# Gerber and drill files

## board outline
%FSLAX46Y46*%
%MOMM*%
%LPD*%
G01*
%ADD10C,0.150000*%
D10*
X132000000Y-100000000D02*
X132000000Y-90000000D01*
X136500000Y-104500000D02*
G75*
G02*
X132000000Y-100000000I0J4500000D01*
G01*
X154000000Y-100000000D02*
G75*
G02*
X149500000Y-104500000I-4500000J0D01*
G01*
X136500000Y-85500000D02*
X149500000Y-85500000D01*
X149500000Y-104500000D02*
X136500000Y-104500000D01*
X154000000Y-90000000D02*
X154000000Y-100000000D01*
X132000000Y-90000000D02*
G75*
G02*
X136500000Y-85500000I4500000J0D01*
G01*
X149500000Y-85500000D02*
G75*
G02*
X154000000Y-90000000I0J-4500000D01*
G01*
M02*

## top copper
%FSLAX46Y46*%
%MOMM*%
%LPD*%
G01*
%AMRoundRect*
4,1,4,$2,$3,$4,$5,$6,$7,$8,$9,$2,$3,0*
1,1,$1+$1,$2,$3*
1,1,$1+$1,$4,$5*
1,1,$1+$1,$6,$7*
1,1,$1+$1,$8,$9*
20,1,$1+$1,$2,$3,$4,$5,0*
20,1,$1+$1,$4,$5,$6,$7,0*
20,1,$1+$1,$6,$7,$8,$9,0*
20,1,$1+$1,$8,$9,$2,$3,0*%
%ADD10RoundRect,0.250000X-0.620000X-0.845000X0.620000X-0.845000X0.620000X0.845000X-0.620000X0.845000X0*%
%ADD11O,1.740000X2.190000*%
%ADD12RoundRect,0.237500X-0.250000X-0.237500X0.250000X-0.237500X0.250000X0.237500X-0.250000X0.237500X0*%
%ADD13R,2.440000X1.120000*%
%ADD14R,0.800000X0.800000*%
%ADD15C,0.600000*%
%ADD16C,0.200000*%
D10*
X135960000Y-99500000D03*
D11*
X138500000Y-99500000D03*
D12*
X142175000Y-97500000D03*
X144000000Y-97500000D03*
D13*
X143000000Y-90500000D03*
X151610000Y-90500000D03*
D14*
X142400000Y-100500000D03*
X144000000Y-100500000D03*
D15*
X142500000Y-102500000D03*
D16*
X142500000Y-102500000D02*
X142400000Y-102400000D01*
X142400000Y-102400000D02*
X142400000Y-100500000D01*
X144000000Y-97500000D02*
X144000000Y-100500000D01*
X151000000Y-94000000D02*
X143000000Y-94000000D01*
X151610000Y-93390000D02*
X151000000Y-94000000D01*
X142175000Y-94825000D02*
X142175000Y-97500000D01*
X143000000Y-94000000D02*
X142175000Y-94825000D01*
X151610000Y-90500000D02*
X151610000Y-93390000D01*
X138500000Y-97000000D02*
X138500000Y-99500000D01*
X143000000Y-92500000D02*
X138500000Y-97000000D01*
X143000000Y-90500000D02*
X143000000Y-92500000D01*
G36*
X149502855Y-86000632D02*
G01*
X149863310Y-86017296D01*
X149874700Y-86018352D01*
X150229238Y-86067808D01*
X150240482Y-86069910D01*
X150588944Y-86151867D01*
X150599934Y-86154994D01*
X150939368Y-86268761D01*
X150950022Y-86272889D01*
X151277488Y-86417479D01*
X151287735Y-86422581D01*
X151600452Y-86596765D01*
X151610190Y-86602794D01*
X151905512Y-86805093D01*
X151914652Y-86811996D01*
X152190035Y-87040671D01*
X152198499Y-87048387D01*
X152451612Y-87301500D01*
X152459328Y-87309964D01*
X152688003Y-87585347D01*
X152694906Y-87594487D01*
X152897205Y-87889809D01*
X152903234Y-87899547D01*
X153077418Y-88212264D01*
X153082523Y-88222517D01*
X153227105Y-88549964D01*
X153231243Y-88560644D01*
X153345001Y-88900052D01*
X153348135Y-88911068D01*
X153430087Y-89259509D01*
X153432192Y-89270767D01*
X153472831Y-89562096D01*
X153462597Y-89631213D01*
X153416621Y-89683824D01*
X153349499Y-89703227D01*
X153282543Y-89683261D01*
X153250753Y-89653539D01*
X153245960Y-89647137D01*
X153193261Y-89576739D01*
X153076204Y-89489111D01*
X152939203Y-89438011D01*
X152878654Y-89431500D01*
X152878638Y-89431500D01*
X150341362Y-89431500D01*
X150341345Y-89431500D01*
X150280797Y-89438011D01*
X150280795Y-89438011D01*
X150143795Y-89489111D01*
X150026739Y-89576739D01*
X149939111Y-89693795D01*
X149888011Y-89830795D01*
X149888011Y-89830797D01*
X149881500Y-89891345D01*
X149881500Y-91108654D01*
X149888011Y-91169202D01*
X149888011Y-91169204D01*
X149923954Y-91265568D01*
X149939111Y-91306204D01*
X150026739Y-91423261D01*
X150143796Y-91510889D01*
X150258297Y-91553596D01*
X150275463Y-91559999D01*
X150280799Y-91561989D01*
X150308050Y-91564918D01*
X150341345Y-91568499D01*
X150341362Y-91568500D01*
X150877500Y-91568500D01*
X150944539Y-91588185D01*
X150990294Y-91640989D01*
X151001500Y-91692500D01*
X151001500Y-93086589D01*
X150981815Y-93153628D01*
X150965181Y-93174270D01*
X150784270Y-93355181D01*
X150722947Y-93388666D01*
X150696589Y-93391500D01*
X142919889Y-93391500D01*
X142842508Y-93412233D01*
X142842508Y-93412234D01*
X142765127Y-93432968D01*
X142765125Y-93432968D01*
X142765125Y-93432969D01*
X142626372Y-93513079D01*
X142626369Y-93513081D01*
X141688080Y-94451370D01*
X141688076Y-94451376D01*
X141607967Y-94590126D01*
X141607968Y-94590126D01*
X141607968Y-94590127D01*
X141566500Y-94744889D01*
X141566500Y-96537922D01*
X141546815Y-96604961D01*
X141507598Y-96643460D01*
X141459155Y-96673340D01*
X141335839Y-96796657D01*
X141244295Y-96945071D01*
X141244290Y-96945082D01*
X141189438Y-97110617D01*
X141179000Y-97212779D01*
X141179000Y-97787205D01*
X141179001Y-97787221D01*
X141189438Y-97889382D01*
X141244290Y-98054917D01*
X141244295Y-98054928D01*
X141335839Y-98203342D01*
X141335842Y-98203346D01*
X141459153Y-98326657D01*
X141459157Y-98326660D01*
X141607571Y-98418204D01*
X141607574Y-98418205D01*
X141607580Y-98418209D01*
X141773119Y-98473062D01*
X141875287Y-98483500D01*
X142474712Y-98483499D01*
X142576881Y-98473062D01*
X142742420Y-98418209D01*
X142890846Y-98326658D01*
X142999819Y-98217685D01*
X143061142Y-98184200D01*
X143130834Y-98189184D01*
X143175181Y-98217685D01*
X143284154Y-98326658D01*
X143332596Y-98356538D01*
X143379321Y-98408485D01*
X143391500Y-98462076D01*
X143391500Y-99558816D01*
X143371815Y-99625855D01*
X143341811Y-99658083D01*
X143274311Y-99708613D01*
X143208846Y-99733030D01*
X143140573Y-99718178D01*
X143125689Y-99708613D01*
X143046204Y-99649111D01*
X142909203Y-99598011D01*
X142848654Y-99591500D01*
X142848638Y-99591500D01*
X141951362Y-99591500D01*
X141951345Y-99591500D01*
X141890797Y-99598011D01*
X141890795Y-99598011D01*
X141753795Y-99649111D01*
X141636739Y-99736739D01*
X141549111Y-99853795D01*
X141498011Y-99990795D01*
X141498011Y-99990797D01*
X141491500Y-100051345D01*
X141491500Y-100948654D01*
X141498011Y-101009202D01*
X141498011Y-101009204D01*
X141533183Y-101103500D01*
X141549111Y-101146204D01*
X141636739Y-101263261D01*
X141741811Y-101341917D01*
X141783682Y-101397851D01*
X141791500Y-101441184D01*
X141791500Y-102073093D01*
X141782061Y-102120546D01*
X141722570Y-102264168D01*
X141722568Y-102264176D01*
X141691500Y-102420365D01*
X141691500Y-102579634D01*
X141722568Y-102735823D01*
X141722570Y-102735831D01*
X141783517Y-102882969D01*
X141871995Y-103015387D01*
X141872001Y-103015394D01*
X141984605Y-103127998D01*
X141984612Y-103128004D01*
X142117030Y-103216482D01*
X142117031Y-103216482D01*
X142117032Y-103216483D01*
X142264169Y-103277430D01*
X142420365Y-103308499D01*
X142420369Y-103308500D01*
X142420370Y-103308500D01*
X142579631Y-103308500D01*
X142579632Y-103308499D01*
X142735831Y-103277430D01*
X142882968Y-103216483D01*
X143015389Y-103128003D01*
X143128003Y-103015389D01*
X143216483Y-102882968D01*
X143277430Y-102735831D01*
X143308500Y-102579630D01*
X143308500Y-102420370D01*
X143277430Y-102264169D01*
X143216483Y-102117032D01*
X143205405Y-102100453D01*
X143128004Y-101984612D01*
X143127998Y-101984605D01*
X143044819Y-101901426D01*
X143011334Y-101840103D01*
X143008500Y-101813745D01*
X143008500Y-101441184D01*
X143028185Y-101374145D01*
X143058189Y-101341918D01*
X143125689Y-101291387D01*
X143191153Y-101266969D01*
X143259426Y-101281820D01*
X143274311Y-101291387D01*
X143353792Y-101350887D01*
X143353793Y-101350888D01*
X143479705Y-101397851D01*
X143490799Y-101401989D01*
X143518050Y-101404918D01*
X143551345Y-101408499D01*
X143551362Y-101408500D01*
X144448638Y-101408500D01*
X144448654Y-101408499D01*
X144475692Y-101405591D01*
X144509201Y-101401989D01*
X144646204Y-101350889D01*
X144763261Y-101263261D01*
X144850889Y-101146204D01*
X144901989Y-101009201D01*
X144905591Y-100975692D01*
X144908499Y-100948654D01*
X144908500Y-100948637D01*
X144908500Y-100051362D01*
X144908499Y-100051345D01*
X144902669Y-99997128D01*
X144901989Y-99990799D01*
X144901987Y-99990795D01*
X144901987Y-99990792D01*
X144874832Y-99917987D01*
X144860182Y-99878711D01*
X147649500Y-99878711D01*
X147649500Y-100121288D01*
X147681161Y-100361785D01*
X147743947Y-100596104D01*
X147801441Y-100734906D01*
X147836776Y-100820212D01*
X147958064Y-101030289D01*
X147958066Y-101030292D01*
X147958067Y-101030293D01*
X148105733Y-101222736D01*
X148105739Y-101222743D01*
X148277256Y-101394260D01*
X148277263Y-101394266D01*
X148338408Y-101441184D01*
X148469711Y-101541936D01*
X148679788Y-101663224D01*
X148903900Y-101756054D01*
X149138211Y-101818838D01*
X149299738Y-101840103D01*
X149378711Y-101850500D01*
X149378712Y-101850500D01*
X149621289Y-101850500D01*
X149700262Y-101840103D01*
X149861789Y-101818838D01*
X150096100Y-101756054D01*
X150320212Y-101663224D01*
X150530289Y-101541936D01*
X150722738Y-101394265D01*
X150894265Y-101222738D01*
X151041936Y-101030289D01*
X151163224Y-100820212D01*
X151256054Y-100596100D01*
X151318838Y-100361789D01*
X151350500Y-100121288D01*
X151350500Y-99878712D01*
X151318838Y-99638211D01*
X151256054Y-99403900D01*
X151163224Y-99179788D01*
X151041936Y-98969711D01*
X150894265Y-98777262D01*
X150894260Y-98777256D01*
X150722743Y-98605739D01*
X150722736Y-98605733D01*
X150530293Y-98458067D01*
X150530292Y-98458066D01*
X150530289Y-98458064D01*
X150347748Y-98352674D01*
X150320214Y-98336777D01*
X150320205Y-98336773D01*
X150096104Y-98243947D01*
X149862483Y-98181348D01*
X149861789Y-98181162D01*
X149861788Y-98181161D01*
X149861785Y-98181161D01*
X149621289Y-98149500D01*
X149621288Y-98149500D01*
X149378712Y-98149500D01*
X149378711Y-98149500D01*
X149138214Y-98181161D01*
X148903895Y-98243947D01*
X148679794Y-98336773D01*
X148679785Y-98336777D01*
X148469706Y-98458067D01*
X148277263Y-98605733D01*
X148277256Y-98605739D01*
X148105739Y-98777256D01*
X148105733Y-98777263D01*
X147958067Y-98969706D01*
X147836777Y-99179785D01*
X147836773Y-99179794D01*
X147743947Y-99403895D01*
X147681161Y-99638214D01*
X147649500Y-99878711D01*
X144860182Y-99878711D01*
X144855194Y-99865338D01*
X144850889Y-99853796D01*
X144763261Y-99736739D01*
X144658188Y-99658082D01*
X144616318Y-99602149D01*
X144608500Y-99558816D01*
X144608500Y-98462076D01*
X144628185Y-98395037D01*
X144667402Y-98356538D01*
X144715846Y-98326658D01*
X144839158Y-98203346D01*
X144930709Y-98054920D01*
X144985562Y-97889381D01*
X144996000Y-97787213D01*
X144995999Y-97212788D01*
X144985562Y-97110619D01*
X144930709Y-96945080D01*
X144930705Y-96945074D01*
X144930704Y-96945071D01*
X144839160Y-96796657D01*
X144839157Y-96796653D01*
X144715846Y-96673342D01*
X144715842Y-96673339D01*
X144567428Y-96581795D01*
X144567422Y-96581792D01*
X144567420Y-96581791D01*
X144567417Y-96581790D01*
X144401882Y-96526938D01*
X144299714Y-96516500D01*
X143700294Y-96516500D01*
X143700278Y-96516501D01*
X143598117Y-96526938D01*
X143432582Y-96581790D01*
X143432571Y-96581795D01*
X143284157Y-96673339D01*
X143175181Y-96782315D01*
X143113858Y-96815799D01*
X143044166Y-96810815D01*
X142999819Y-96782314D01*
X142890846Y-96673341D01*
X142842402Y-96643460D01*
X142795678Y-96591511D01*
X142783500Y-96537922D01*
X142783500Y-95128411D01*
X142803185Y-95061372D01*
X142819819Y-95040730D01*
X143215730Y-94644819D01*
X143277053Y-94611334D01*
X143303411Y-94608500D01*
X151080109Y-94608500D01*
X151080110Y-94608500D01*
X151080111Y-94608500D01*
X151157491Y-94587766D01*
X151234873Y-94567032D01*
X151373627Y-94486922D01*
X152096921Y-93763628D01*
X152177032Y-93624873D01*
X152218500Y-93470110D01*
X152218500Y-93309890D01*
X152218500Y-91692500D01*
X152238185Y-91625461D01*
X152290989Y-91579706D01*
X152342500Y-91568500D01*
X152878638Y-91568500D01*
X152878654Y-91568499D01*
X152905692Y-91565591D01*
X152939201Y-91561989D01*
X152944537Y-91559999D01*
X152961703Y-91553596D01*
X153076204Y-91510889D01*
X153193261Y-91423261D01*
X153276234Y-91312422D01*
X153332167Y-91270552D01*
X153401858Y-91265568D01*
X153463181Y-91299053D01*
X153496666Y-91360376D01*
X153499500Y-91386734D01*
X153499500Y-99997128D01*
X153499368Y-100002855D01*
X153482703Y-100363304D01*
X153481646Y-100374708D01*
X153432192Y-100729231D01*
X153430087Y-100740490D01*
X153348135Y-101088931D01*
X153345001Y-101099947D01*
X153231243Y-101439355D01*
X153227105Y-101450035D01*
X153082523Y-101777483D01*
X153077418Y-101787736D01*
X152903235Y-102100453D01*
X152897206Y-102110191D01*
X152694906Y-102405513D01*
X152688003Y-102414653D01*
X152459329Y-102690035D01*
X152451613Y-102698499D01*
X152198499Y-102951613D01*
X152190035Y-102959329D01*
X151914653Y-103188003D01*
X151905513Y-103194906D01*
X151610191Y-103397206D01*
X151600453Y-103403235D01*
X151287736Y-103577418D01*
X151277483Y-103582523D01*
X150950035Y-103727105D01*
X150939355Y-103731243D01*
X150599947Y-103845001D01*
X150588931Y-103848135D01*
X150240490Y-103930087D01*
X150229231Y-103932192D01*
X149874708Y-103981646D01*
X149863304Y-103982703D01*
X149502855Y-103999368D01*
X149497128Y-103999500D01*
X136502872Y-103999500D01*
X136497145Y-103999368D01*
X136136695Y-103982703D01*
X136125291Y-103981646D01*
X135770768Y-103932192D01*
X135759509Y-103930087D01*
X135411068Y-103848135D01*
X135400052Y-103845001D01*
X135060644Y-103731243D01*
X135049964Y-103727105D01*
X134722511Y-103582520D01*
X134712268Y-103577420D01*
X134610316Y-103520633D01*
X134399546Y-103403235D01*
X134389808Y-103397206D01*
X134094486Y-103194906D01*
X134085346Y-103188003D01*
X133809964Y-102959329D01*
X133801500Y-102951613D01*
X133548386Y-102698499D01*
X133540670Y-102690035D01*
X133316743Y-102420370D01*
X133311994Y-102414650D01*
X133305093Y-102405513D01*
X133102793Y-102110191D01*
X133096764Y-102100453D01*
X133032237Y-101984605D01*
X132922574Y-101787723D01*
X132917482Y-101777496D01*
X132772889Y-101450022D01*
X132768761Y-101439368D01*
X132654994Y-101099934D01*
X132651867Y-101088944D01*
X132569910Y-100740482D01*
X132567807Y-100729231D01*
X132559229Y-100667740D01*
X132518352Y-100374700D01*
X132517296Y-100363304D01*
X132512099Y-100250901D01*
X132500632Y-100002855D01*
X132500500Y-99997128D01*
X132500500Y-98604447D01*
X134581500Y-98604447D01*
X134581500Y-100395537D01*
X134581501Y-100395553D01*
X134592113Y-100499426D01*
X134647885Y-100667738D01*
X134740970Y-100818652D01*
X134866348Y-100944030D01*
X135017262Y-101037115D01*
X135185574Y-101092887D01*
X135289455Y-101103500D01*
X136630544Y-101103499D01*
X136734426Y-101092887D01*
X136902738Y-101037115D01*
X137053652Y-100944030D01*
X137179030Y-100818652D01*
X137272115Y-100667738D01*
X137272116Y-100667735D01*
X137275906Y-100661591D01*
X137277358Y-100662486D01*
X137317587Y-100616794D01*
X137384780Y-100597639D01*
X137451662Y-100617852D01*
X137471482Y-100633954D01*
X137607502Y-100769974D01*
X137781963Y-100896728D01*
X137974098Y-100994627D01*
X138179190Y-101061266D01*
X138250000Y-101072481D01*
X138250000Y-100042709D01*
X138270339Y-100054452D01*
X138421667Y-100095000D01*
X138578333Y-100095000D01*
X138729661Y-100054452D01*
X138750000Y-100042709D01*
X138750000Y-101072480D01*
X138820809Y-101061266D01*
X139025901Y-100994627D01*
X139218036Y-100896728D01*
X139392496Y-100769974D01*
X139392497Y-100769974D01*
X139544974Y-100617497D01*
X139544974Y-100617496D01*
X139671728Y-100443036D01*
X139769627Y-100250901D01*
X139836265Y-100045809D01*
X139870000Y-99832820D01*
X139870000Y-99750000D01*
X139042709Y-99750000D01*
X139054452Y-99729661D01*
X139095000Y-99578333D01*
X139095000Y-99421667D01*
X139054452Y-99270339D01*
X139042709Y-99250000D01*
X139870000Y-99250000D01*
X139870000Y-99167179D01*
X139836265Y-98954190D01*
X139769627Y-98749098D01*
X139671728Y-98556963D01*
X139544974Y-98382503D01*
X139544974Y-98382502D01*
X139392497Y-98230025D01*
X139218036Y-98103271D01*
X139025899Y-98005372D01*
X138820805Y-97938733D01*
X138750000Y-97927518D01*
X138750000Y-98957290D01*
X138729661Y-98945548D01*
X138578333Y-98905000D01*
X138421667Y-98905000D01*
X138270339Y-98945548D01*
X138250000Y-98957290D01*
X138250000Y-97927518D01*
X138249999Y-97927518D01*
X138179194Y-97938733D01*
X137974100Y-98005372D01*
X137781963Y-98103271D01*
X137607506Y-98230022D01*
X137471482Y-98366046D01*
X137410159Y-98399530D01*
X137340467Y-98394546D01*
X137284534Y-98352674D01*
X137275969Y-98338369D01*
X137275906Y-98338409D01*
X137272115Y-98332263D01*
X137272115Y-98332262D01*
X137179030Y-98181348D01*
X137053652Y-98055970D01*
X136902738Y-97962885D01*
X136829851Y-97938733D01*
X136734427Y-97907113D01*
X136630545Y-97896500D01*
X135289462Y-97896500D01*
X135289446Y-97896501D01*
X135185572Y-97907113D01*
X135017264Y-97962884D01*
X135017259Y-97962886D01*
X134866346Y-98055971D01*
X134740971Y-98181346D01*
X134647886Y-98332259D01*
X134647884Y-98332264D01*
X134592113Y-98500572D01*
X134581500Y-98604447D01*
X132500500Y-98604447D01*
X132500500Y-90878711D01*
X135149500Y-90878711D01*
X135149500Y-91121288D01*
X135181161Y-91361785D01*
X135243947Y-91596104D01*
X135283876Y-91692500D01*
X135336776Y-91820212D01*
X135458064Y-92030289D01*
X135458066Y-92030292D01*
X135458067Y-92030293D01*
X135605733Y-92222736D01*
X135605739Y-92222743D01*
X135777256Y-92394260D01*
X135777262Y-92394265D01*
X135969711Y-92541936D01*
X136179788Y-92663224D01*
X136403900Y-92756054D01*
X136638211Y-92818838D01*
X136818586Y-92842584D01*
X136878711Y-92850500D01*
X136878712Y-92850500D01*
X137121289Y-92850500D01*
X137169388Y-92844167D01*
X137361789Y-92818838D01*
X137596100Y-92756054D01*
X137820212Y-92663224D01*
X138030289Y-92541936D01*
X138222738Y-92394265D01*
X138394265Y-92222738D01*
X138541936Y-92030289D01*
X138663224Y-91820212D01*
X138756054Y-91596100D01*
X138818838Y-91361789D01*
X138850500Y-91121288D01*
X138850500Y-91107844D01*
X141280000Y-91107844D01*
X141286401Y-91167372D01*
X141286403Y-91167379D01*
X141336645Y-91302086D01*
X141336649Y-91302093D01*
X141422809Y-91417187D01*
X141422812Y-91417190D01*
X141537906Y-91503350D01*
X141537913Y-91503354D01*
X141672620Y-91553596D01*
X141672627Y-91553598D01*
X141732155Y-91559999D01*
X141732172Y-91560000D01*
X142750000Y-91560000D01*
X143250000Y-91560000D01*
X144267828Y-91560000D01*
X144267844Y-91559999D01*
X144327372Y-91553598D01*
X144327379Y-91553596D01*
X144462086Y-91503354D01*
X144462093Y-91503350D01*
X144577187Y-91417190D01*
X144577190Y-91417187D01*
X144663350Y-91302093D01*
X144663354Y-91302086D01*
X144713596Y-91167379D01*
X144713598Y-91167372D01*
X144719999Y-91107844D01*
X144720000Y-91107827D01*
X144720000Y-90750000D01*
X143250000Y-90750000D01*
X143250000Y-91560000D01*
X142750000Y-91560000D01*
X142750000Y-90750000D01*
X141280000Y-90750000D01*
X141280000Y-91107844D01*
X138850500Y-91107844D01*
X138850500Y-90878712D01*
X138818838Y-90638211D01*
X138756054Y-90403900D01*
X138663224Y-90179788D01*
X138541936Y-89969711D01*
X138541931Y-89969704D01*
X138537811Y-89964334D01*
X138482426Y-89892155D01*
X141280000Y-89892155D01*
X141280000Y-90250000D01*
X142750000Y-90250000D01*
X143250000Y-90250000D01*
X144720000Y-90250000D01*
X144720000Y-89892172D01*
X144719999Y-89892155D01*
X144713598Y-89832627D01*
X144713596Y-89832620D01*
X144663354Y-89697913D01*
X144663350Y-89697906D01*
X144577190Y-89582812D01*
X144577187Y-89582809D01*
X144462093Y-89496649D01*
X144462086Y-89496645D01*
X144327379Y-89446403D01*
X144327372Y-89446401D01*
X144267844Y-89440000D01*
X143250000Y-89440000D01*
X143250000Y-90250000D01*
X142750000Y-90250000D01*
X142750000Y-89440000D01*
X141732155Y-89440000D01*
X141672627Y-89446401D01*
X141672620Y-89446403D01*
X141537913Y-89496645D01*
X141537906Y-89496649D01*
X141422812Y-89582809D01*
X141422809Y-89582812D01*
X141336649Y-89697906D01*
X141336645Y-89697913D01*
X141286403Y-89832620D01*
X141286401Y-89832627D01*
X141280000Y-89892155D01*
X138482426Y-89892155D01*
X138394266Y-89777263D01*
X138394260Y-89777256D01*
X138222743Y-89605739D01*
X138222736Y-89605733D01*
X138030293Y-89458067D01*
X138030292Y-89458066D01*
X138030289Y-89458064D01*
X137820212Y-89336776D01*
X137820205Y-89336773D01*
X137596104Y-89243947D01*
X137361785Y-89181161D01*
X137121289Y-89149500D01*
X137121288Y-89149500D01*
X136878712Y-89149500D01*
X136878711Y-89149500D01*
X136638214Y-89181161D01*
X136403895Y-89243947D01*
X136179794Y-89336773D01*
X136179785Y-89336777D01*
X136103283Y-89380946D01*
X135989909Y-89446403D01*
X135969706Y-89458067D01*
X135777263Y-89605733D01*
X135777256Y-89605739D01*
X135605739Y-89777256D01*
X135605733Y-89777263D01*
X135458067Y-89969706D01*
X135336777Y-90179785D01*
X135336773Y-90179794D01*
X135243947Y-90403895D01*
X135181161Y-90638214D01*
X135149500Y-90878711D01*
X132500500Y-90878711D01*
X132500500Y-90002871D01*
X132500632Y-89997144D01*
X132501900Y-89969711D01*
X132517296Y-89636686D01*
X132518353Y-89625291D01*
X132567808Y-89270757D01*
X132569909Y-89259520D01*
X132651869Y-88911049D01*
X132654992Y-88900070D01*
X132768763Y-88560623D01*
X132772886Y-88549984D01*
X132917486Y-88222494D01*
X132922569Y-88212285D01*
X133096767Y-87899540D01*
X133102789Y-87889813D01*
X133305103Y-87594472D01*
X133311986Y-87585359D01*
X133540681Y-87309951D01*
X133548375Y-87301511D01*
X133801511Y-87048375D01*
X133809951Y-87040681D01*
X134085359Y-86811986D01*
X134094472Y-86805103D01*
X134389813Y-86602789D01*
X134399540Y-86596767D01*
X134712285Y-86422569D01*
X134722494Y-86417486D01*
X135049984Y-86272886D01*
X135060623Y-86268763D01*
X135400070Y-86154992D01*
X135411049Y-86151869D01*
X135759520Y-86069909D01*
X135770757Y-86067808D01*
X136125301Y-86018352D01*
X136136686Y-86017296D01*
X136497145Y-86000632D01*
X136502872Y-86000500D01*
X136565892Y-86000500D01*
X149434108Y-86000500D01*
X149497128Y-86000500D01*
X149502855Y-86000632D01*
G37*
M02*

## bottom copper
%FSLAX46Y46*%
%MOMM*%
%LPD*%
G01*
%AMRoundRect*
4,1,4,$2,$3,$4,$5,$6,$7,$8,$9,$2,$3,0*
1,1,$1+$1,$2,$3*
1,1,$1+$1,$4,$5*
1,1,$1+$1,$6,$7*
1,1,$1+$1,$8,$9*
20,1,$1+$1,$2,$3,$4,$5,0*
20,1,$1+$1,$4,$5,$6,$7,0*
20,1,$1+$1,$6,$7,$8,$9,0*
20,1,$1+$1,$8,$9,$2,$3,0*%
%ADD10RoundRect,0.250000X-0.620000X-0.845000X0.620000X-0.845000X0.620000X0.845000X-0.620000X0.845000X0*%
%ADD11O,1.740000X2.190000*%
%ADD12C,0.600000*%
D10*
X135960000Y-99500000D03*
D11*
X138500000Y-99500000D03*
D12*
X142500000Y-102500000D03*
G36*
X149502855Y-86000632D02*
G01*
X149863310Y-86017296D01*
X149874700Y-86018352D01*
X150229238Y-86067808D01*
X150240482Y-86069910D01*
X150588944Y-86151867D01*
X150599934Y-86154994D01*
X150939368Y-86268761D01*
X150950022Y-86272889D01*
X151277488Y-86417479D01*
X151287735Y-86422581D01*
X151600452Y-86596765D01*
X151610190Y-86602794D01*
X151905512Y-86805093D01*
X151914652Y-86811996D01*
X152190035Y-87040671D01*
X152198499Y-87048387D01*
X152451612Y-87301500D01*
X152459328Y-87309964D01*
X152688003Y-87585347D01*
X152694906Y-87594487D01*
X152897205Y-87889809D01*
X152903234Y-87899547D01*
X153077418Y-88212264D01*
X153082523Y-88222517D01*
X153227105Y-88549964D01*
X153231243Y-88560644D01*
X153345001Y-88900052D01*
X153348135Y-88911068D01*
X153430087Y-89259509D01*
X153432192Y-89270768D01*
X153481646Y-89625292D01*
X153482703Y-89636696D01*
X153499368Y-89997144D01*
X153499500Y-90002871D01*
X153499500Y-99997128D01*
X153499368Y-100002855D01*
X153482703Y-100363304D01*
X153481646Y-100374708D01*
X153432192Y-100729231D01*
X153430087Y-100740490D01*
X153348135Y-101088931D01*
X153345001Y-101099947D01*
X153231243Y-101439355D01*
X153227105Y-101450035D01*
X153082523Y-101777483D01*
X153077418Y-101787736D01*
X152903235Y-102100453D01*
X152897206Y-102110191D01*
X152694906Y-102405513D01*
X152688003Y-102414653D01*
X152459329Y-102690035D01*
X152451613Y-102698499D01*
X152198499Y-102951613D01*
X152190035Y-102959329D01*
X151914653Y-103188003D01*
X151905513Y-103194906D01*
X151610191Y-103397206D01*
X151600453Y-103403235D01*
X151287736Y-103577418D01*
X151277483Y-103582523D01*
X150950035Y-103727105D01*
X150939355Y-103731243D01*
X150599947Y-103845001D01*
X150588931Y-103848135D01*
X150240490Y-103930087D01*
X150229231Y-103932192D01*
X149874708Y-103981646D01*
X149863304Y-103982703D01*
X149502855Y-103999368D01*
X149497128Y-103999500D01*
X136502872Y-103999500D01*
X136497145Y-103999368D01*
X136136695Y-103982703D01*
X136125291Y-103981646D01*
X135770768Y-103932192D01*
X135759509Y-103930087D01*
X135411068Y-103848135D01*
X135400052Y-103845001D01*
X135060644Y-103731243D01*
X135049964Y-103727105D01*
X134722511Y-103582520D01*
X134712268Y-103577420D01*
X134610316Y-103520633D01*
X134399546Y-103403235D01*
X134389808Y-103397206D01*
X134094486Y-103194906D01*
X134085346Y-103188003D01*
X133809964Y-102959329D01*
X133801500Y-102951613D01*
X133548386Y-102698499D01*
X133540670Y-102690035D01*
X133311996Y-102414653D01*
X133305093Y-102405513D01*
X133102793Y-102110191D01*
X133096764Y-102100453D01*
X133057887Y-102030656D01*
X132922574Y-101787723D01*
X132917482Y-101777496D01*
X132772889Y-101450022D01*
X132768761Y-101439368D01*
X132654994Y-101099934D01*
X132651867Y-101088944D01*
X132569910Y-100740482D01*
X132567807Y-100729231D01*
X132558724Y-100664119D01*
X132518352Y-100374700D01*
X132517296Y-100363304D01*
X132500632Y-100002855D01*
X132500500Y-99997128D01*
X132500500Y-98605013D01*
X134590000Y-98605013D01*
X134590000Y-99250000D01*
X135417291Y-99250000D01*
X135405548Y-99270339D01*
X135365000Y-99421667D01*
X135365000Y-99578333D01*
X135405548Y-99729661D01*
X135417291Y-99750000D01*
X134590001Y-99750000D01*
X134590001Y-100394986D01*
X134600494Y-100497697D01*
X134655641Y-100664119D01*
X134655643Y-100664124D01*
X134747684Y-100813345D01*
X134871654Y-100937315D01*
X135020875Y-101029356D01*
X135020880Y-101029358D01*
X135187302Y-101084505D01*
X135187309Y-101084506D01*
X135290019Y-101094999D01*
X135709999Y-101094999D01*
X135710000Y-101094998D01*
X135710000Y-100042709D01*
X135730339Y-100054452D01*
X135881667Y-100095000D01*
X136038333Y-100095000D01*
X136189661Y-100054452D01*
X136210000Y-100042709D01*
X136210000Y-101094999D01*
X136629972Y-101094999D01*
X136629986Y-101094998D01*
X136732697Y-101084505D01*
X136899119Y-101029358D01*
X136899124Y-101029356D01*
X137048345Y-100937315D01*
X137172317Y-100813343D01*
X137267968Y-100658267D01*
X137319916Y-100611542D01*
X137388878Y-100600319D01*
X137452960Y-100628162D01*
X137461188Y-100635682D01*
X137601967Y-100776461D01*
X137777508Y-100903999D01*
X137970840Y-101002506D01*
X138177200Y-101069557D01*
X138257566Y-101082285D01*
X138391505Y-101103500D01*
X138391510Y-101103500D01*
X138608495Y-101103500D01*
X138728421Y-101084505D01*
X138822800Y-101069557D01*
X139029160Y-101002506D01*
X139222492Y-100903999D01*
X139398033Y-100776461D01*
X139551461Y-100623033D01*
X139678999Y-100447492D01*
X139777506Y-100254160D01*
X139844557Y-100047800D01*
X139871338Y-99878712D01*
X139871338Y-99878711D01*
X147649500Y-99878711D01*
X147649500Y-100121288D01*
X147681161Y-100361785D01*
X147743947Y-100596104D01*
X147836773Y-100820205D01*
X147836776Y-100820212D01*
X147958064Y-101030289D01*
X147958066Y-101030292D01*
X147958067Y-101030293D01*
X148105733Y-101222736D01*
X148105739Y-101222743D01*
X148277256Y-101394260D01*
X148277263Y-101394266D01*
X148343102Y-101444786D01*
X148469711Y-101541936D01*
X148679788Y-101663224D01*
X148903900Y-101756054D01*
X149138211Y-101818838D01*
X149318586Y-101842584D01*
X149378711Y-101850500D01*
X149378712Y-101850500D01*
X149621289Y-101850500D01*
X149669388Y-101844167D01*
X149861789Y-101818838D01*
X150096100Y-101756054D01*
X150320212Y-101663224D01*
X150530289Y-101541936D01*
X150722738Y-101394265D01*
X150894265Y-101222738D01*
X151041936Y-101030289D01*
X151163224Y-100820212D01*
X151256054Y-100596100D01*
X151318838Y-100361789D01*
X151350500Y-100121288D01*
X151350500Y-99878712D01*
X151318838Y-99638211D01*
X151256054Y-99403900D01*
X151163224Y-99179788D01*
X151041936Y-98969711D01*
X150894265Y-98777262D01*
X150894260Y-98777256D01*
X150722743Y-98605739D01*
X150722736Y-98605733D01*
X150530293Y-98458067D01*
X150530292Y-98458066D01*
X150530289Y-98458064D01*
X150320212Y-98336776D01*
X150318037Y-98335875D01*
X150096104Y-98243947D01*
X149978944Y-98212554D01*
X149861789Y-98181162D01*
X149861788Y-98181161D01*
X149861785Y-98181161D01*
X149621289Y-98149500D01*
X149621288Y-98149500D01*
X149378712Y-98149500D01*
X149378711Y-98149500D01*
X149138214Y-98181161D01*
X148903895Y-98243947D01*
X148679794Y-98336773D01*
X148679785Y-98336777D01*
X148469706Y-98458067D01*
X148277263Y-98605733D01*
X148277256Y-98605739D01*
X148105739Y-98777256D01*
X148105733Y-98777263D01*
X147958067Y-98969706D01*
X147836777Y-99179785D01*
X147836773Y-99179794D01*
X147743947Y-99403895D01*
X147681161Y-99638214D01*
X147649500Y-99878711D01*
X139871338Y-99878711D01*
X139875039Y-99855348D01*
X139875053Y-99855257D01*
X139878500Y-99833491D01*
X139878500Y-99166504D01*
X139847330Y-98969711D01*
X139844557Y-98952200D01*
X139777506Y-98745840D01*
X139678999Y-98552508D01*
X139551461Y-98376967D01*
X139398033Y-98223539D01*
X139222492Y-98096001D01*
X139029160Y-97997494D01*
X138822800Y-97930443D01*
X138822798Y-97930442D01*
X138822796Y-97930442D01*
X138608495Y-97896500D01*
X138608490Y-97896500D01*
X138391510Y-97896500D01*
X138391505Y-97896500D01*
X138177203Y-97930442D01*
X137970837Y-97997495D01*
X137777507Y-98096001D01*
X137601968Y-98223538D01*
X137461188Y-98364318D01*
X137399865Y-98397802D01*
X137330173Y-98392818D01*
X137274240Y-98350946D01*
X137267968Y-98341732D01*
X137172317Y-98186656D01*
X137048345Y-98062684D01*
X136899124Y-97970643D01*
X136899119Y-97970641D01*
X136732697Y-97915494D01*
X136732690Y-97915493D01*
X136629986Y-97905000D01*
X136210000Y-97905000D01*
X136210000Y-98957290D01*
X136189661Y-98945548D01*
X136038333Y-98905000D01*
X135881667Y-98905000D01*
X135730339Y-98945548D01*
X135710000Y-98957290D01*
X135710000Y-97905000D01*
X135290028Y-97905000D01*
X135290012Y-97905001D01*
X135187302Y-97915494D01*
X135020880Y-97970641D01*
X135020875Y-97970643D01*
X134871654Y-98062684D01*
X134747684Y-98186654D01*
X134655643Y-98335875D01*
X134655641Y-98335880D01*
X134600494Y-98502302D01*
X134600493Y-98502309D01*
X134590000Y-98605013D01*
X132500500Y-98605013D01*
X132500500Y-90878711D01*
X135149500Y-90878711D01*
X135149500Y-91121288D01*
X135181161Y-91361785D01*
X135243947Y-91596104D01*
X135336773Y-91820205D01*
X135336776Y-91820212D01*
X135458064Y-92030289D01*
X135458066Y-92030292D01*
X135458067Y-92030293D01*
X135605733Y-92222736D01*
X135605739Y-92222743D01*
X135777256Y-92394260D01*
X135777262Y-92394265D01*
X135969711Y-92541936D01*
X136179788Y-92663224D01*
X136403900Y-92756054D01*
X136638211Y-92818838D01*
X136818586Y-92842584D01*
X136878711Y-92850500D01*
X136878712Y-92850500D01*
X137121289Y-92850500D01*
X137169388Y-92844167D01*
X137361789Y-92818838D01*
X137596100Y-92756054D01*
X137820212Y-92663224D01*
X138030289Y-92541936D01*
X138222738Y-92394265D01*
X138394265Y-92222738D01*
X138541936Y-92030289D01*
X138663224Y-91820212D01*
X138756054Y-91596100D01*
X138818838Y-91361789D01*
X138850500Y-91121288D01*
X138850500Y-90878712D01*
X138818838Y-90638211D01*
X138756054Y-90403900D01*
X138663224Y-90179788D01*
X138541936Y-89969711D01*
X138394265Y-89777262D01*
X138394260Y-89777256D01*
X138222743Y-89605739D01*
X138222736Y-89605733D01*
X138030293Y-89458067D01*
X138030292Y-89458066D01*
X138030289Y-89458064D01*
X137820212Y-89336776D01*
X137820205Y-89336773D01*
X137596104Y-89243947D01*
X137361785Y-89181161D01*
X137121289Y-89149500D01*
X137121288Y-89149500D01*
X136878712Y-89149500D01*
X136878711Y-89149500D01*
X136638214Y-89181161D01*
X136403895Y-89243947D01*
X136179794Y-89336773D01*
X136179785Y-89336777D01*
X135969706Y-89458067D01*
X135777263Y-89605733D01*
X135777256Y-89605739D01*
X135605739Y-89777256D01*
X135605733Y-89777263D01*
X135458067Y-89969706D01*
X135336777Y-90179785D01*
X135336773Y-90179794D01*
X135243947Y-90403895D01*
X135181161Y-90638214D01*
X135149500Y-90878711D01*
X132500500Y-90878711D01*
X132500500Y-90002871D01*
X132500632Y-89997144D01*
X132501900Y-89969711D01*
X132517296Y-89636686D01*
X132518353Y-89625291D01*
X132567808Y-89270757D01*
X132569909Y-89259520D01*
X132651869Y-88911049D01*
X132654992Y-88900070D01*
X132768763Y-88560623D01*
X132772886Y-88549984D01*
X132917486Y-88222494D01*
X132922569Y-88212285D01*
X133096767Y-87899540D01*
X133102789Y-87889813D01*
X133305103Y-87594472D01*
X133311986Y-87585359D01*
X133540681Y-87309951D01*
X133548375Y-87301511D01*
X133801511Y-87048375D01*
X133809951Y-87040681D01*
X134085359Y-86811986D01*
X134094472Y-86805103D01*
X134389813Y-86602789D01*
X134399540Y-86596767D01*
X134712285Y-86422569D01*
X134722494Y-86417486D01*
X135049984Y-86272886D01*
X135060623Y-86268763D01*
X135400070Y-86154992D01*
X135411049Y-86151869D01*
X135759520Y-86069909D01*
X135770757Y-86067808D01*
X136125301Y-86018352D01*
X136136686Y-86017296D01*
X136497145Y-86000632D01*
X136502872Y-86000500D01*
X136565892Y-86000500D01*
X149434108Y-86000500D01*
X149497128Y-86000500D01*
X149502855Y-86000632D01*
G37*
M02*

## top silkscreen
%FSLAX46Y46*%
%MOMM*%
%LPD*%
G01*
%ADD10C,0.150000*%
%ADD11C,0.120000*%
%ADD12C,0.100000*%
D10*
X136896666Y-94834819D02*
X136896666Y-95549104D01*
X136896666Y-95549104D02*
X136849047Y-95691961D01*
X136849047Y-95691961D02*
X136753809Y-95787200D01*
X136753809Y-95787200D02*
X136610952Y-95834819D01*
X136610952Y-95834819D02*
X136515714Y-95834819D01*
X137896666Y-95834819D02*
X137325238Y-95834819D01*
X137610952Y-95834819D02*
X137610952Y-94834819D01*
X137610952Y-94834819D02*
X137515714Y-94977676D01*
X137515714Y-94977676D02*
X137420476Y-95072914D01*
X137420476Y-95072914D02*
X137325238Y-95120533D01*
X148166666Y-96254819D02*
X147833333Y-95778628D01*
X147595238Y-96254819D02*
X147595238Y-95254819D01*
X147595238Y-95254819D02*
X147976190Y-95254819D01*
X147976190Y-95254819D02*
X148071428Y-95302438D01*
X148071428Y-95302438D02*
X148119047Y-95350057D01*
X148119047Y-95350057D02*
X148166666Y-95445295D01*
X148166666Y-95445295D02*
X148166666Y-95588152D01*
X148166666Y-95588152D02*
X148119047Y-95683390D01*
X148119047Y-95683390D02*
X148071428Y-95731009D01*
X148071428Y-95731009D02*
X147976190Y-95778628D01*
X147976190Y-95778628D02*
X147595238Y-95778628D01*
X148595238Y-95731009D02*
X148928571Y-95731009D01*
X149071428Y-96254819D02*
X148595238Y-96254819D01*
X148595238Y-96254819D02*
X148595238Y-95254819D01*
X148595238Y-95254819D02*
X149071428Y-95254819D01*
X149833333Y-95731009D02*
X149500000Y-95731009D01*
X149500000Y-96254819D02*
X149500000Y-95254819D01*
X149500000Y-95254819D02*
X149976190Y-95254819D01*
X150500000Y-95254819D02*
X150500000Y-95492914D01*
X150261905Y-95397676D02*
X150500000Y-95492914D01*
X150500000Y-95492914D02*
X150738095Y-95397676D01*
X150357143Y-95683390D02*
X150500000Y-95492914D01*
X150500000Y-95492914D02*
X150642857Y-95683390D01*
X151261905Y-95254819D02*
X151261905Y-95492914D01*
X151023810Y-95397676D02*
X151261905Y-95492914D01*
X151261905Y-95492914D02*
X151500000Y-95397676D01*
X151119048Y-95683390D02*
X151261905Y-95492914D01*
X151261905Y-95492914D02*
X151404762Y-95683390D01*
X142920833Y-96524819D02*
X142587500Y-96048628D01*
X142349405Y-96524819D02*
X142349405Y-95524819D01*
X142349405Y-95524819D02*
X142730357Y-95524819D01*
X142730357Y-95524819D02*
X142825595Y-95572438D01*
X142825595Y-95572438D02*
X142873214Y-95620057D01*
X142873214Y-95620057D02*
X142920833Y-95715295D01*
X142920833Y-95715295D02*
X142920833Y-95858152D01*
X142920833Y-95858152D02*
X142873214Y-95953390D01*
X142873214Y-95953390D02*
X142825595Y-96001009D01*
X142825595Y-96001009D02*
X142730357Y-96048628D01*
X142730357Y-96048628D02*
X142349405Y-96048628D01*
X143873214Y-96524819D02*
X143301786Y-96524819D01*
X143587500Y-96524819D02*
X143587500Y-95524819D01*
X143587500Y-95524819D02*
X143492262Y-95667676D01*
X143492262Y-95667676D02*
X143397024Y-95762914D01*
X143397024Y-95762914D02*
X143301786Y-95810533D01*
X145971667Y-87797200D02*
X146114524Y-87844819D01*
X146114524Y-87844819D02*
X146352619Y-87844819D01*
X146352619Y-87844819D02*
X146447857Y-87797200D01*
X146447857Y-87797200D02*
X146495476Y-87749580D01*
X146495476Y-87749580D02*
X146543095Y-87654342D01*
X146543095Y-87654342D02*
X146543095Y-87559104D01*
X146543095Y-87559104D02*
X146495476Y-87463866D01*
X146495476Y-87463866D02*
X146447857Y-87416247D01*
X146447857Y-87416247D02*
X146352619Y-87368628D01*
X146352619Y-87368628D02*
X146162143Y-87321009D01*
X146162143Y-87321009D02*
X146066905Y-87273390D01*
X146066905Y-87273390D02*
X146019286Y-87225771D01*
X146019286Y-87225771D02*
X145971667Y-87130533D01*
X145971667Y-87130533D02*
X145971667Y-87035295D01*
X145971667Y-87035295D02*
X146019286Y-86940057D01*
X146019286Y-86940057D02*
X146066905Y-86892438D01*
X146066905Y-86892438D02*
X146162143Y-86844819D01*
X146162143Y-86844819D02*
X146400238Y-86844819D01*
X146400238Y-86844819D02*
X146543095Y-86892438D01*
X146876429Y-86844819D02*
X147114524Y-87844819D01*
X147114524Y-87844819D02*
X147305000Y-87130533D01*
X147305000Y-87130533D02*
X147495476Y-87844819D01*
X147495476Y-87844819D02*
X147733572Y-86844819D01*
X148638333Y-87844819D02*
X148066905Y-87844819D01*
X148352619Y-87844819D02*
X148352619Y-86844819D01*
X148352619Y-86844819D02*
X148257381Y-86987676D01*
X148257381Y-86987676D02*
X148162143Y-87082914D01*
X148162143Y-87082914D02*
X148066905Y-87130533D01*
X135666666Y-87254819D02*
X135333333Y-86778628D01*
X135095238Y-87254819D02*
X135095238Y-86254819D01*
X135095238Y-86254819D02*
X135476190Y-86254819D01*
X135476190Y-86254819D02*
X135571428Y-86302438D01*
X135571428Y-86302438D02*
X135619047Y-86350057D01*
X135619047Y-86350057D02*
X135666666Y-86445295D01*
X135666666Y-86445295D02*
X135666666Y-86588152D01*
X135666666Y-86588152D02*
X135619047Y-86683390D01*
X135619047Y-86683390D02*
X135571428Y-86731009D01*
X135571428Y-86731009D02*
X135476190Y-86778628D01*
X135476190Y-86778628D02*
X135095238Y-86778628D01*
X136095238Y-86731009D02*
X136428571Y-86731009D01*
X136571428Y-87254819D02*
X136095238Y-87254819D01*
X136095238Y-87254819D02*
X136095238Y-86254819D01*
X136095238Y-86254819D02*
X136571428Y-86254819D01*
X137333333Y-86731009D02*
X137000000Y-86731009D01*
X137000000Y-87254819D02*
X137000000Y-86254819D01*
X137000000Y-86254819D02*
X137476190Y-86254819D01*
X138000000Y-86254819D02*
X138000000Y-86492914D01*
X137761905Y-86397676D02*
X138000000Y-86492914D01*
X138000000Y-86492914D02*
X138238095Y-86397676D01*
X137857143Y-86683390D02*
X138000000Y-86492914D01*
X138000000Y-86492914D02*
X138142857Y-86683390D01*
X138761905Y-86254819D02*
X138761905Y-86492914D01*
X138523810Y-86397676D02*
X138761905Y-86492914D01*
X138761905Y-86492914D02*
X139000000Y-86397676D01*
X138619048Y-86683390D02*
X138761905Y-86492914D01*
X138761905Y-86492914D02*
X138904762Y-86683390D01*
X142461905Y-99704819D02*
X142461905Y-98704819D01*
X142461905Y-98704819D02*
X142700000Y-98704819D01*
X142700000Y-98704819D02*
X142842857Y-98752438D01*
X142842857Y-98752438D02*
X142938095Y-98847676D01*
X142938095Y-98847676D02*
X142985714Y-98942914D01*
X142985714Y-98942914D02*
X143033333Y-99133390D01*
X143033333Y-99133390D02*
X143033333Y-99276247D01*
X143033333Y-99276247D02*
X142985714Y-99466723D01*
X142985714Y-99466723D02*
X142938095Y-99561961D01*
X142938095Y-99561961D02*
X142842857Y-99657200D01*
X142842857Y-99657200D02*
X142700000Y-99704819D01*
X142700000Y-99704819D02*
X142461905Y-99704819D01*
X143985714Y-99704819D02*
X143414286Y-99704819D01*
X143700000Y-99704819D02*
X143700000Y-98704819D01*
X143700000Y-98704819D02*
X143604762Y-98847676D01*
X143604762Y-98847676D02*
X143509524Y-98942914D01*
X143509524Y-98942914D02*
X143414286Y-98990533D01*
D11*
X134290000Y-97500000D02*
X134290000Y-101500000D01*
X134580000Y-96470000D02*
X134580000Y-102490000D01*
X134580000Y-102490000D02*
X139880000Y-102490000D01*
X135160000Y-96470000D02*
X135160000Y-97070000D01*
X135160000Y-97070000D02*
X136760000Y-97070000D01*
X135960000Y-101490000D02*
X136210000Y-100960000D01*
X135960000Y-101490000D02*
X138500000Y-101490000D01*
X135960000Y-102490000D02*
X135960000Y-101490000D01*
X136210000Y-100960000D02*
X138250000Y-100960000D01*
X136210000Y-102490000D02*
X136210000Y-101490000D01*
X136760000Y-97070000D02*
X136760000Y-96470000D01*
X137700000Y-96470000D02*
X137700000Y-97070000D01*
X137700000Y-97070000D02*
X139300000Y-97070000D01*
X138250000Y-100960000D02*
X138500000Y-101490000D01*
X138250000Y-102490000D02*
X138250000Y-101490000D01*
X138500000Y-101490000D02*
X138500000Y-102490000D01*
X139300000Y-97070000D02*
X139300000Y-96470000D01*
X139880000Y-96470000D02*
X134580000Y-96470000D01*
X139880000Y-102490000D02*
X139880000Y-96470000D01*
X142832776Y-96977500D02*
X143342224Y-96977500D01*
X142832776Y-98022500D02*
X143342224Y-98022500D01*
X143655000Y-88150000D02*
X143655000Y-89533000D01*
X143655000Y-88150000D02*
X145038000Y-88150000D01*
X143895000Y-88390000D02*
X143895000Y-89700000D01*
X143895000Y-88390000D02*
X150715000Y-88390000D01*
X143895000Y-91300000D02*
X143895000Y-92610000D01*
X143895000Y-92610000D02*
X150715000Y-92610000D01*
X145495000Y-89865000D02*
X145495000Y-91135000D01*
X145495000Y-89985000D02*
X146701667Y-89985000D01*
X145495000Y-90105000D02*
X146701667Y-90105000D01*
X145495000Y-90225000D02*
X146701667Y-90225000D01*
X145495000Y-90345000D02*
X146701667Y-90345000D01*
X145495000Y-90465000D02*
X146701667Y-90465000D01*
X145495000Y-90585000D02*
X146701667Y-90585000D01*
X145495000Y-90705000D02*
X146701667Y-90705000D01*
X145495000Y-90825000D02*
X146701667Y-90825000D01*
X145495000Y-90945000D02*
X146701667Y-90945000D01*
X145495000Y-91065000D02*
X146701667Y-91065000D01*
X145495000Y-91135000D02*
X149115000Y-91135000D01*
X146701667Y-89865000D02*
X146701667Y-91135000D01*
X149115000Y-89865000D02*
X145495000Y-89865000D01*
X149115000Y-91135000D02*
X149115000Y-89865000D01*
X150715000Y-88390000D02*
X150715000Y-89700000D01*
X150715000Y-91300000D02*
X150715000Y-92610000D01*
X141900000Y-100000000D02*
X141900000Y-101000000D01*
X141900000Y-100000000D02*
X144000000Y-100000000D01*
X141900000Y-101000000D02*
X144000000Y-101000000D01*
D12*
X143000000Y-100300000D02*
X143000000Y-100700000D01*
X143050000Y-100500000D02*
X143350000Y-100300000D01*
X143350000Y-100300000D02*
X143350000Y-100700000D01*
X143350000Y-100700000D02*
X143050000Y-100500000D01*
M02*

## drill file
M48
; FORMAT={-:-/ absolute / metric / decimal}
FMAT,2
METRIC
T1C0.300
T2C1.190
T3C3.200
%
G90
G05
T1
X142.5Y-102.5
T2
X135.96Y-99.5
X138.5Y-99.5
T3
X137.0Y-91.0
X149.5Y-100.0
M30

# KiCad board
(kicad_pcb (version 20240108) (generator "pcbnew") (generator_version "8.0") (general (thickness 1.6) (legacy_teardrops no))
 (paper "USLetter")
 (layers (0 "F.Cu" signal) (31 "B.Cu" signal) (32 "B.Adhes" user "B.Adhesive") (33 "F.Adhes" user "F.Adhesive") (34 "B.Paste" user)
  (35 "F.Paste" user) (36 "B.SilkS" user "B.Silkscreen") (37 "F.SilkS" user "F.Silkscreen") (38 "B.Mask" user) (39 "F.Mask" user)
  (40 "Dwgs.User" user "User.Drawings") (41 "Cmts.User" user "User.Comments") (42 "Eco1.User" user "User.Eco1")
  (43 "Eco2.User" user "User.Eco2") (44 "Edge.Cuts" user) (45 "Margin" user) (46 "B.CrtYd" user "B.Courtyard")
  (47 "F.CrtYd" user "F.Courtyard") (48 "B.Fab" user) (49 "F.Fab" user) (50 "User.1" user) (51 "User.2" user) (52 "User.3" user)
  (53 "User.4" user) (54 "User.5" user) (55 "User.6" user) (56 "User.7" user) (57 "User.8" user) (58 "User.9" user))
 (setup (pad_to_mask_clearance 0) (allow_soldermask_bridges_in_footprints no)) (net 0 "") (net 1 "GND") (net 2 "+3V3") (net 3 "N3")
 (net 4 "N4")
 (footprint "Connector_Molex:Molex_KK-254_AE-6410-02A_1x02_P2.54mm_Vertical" (layer "F.Cu") (at 135.96 99.5)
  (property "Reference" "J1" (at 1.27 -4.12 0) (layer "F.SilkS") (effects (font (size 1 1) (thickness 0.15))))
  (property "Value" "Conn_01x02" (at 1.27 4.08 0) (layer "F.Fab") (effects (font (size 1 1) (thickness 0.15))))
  (fp_line (start -1.67 -2) (end -1.67 2) (stroke (width 0.12) (type solid)) (layer "F.SilkS"))
  (fp_line (start -1.38 -3.03) (end -1.38 2.99) (stroke (width 0.12) (type solid)) (layer "F.SilkS"))
  (fp_line (start -1.38 2.99) (end 3.92 2.99) (stroke (width 0.12) (type solid)) (layer "F.SilkS"))
  (fp_line (start -0.8 -3.03) (end -0.8 -2.43) (stroke (width 0.12) (type solid)) (layer "F.SilkS"))
  (fp_line (start -0.8 -2.43) (end 0.8 -2.43) (stroke (width 0.12) (type solid)) (layer "F.SilkS"))
  (fp_line (start 0 1.99) (end 0.25 1.46) (stroke (width 0.12) (type solid)) (layer "F.SilkS"))
  (fp_line (start 0 1.99) (end 2.54 1.99) (stroke (width 0.12) (type solid)) (layer "F.SilkS"))
  (fp_line (start 0 2.99) (end 0 1.99) (stroke (width 0.12) (type solid)) (layer "F.SilkS"))
  (fp_line (start 0.25 1.46) (end 2.29 1.46) (stroke (width 0.12) (type solid)) (layer "F.SilkS"))
  (fp_line (start 0.25 2.99) (end 0.25 1.99) (stroke (width 0.12) (type solid)) (layer "F.SilkS"))
  (fp_line (start 0.8 -2.43) (end 0.8 -3.03) (stroke (width 0.12) (type solid)) (layer "F.SilkS"))
  (fp_line (start 1.74 -3.03) (end 1.74 -2.43) (stroke (width 0.12) (type solid)) (layer "F.SilkS"))
  (fp_line (start 1.74 -2.43) (end 3.34 -2.43) (stroke (width 0.12) (type solid)) (layer "F.SilkS"))
  (fp_line (start 2.29 1.46) (end 2.54 1.99) (stroke (width 0.12) (type solid)) (layer "F.SilkS"))
  (fp_line (start 2.29 2.99) (end 2.29 1.99) (stroke (width 0.12) (type solid)) (layer "F.SilkS"))
  (fp_line (start 2.54 1.99) (end 2.54 2.99) (stroke (width 0.12) (type solid)) (layer "F.SilkS"))
  (fp_line (start 3.34 -2.43) (end 3.34 -3.03) (stroke (width 0.12) (type solid)) (layer "F.SilkS"))
  (fp_line (start 3.92 -3.03) (end -1.38 -3.03) (stroke (width 0.12) (type solid)) (layer "F.SilkS"))
  (fp_line (start 3.92 2.99) (end 3.92 -3.03) (stroke (width 0.12) (type solid)) (layer "F.SilkS"))
  (pad "1" thru_hole roundrect (at 0 0) (size 1.74 2.19) (drill 1.19) (layers "*.Cu" "*.Mask") (remove_unused_layers no)
   (roundrect_rratio 0.143678) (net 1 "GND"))
  (pad "2" thru_hole oval (at 2.54 0) (size 1.74 2.19) (drill 1.19) (layers "*.Cu" "*.Mask") (remove_unused_layers no) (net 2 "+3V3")))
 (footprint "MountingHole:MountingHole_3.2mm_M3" (layer "F.Cu") (at 149.5 100)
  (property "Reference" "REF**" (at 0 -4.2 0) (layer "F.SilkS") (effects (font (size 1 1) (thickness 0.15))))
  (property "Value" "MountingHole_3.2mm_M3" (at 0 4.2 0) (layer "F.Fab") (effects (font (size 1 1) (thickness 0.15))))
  (pad "" np_thru_hole circle (at 0 0) (size 3.2 3.2) (drill 3.2) (layers "*.Cu" "*.Mask")))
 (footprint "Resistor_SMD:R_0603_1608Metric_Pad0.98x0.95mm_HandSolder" (layer "F.Cu") (at 143.0875 97.5)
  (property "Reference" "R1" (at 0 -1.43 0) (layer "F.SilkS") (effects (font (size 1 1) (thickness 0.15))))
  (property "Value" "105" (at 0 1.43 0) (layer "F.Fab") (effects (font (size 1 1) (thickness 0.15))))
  (fp_line (start -0.254724 -0.5225) (end 0.254724 -0.5225) (stroke (width 0.12) (type solid)) (layer "F.SilkS"))
  (fp_line (start -0.254724 0.5225) (end 0.254724 0.5225) (stroke (width 0.12) (type solid)) (layer "F.SilkS"))
  (pad "1" smd roundrect (at -0.9125 0) (size 0.975 0.95) (layers "F.Cu" "F.Paste" "F.Mask") (roundrect_rratio 0.25) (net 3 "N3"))
  (pad "2" smd roundrect (at 0.9125 0) (size 0.975 0.95) (layers "F.Cu" "F.Paste" "F.Mask") (roundrect_rratio 0.25) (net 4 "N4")))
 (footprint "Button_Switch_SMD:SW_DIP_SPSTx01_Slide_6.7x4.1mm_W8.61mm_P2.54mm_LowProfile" (layer "F.Cu") (at 147.305 90.5)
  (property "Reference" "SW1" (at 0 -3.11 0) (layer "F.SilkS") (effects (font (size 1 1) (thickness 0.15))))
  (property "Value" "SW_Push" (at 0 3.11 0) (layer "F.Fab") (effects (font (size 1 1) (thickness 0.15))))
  (fp_line (start -3.65 -2.35) (end -3.65 -0.967) (stroke (width 0.12) (type solid)) (layer "F.SilkS"))
  (fp_line (start -3.65 -2.35) (end -2.267 -2.35) (stroke (width 0.12) (type solid)) (layer "F.SilkS"))
  (fp_line (start -3.41 -2.11) (end -3.41 -0.8) (stroke (width 0.12) (type solid)) (layer "F.SilkS"))
  (fp_line (start -3.41 -2.11) (end 3.41 -2.11) (stroke (width 0.12) (type solid)) (layer "F.SilkS"))
  (fp_line (start -3.41 0.8) (end -3.41 2.11) (stroke (width 0.12) (type solid)) (layer "F.SilkS"))
  (fp_line (start -3.41 2.11) (end 3.41 2.11) (stroke (width 0.12) (type solid)) (layer "F.SilkS"))
  (fp_line (start -1.81 -0.635) (end -1.81 0.635) (stroke (width 0.12) (type solid)) (layer "F.SilkS"))
  (fp_line (start -1.81 -0.515) (end -0.603333 -0.515) (stroke (width 0.12) (type solid)) (layer "F.SilkS"))
  (fp_line (start -1.81 -0.395) (end -0.603333 -0.395) (stroke (width 0.12) (type solid)) (layer "F.SilkS"))
  (fp_line (start -1.81 -0.275) (end -0.603333 -0.275) (stroke (width 0.12) (type solid)) (layer "F.SilkS"))
  (fp_line (start -1.81 -0.155) (end -0.603333 -0.155) (stroke (width 0.12) (type solid)) (layer "F.SilkS"))
  (fp_line (start -1.81 -0.035) (end -0.603333 -0.035) (stroke (width 0.12) (type solid)) (layer "F.SilkS"))
  (fp_line (start -1.81 0.085) (end -0.603333 0.085) (stroke (width 0.12) (type solid)) (layer "F.SilkS"))
  (fp_line (start -1.81 0.205) (end -0.603333 0.205) (stroke (width 0.12) (type solid)) (layer "F.SilkS"))
  (fp_line (start -1.81 0.325) (end -0.603333 0.325) (stroke (width 0.12) (type solid)) (layer "F.SilkS"))
  (fp_line (start -1.81 0.445) (end -0.603333 0.445) (stroke (width 0.12) (type solid)) (layer "F.SilkS"))
  (fp_line (start -1.81 0.565) (end -0.603333 0.565) (stroke (width 0.12) (type solid)) (layer "F.SilkS"))
  (fp_line (start -1.81 0.635) (end 1.81 0.635) (stroke (width 0.12) (type solid)) (layer "F.SilkS"))
  (fp_line (start -0.603333 -0.635) (end -0.603333 0.635) (stroke (width 0.12) (type solid)) (layer "F.SilkS"))
  (fp_line (start 1.81 -0.635) (end -1.81 -0.635) (stroke (width 0.12) (type solid)) (layer "F.SilkS"))
  (fp_line (start 1.81 0.635) (end 1.81 -0.635) (stroke (width 0.12) (type solid)) (layer "F.SilkS"))
  (fp_line (start 3.41 -2.11) (end 3.41 -0.8) (stroke (width 0.12) (type solid)) (layer "F.SilkS"))
  (fp_line (start 3.41 0.8) (end 3.41 2.11) (stroke (width 0.12) (type solid)) (layer "F.SilkS"))
  (pad "1" smd rect (at -4.305 0) (size 2.44 1.12) (layers "F.Cu" "F.Paste" "F.Mask") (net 2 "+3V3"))
  (pad "2" smd rect (at 4.305 0) (size 2.44 1.12) (layers "F.Cu" "F.Paste" "F.Mask") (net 3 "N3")))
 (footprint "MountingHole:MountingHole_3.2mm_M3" (layer "F.Cu") (at 137 91)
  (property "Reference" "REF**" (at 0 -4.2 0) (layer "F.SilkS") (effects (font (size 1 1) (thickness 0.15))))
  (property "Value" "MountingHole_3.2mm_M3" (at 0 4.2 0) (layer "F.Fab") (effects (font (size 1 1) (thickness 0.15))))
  (pad "" np_thru_hole circle (at 0 0) (size 3.2 3.2) (drill 3.2) (layers "*.Cu" "*.Mask")))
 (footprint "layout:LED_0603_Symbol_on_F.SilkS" (layer "F.Cu") (at 143.2 100.5)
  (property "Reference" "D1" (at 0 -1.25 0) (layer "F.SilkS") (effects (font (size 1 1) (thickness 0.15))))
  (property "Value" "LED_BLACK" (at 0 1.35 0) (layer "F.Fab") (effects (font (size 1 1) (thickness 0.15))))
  (fp_line (start -1.3 -0.5) (end -1.3 0.5) (stroke (width 0.12) (type solid)) (layer "F.SilkS"))
  (fp_line (start -1.3 -0.5) (end 0.8 -0.5) (stroke (width 0.12) (type solid)) (layer "F.SilkS"))
  (fp_line (start -1.3 0.5) (end 0.8 0.5) (stroke (width 0.12) (type solid)) (layer "F.SilkS"))
  (fp_line (start -0.2 -0.2) (end -0.2 0.2) (stroke (width 0.1) (type solid)) (layer "F.SilkS"))
  (fp_line (start -0.15 0) (end 0.15 -0.2) (stroke (width 0.1) (type solid)) (layer "F.SilkS"))
  (fp_line (start 0.15 -0.2) (end 0.15 0.2) (stroke (width 0.1) (type solid)) (layer "F.SilkS"))
  (fp_line (start 0.15 0.2) (end -0.15 0) (stroke (width 0.1) (type solid)) (layer "F.SilkS"))
  (pad "1" smd rect (at -0.8 0 180) (size 0.8 0.8) (layers "F.Cu" "F.Paste" "F.Mask") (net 1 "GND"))
  (pad "2" smd rect (at 0.8 0 180) (size 0.8 0.8) (layers "F.Cu" "F.Paste" "F.Mask") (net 4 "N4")))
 (gr_line (start 132 100) (end 132 90) (stroke (width 0.15) (type default)) (layer "Edge.Cuts"))
 (gr_arc (start 136.5 104.5) (mid 133.318019 103.181981) (end 132 100) (stroke (width 0.15) (type default)) (layer "Edge.Cuts"))
 (gr_arc (start 154 100) (mid 152.681981 103.181981) (end 149.5 104.5) (stroke (width 0.15) (type default)) (layer "Edge.Cuts"))
 (gr_line (start 136.5 85.5) (end 149.5 85.5) (stroke (width 0.15) (type default)) (layer "Edge.Cuts"))
 (gr_line (start 149.5 104.5) (end 136.5 104.5) (stroke (width 0.15) (type default)) (layer "Edge.Cuts"))
 (gr_line (start 154 90) (end 154 100) (stroke (width 0.15) (type default)) (layer "Edge.Cuts"))
 (gr_arc (start 132 90) (mid 133.318019 86.818019) (end 136.5 85.5) (stroke (width 0.15) (type default)) (layer "Edge.Cuts"))
 (gr_arc (start 149.5 85.5) (mid 152.68198 86.818019) (end 154 90) (stroke (width 0.15) (type default)) (layer "Edge.Cuts"))
 (segment (start 142.5 102.5) (end 142.4 102.4) (width 0.2) (layer "F.Cu") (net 1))
 (segment (start 142.4 102.4) (end 142.4 100.5) (width 0.2) (layer "F.Cu") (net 1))
 (via (at 142.5 102.5) (size 0.6) (drill 0.3) (layers "F.Cu" "B.Cu") (free yes) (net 1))
 (segment (start 144 97.5) (end 144 100.5) (width 0.2) (layer "F.Cu") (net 4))
 (segment (start 151 94) (end 143 94) (width 0.2) (layer "F.Cu") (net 3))
 (segment (start 151.61 93.39) (end 151 94) (width 0.2) (layer "F.Cu") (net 3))
 (segment (start 142.175 94.825) (end 142.175 97.5) (width 0.2) (layer "F.Cu") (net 3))
 (segment (start 143 94) (end 142.175 94.825) (width 0.2) (layer "F.Cu") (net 3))
 (segment (start 151.61 90.5) (end 151.61 93.39) (width 0.2) (layer "F.Cu") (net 3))
 (segment (start 138.5 97) (end 138.5 99.5) (width 0.2) (layer "F.Cu") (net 2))
 (segment (start 143 92.5) (end 138.5 97) (width 0.2) (layer "F.Cu") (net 2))
 (segment (start 143 90.5) (end 143 92.5) (width 0.2) (layer "F.Cu") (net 2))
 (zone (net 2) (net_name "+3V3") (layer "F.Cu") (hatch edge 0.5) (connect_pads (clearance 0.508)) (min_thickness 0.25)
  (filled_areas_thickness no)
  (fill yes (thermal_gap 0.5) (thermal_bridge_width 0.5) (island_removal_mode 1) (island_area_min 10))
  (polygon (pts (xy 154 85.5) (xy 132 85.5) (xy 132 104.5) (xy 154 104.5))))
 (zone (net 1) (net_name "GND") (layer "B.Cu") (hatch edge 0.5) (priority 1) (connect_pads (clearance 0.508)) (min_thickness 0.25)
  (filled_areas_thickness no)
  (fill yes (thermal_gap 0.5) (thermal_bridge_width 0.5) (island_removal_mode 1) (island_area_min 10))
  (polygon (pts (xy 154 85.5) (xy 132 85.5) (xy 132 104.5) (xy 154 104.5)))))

